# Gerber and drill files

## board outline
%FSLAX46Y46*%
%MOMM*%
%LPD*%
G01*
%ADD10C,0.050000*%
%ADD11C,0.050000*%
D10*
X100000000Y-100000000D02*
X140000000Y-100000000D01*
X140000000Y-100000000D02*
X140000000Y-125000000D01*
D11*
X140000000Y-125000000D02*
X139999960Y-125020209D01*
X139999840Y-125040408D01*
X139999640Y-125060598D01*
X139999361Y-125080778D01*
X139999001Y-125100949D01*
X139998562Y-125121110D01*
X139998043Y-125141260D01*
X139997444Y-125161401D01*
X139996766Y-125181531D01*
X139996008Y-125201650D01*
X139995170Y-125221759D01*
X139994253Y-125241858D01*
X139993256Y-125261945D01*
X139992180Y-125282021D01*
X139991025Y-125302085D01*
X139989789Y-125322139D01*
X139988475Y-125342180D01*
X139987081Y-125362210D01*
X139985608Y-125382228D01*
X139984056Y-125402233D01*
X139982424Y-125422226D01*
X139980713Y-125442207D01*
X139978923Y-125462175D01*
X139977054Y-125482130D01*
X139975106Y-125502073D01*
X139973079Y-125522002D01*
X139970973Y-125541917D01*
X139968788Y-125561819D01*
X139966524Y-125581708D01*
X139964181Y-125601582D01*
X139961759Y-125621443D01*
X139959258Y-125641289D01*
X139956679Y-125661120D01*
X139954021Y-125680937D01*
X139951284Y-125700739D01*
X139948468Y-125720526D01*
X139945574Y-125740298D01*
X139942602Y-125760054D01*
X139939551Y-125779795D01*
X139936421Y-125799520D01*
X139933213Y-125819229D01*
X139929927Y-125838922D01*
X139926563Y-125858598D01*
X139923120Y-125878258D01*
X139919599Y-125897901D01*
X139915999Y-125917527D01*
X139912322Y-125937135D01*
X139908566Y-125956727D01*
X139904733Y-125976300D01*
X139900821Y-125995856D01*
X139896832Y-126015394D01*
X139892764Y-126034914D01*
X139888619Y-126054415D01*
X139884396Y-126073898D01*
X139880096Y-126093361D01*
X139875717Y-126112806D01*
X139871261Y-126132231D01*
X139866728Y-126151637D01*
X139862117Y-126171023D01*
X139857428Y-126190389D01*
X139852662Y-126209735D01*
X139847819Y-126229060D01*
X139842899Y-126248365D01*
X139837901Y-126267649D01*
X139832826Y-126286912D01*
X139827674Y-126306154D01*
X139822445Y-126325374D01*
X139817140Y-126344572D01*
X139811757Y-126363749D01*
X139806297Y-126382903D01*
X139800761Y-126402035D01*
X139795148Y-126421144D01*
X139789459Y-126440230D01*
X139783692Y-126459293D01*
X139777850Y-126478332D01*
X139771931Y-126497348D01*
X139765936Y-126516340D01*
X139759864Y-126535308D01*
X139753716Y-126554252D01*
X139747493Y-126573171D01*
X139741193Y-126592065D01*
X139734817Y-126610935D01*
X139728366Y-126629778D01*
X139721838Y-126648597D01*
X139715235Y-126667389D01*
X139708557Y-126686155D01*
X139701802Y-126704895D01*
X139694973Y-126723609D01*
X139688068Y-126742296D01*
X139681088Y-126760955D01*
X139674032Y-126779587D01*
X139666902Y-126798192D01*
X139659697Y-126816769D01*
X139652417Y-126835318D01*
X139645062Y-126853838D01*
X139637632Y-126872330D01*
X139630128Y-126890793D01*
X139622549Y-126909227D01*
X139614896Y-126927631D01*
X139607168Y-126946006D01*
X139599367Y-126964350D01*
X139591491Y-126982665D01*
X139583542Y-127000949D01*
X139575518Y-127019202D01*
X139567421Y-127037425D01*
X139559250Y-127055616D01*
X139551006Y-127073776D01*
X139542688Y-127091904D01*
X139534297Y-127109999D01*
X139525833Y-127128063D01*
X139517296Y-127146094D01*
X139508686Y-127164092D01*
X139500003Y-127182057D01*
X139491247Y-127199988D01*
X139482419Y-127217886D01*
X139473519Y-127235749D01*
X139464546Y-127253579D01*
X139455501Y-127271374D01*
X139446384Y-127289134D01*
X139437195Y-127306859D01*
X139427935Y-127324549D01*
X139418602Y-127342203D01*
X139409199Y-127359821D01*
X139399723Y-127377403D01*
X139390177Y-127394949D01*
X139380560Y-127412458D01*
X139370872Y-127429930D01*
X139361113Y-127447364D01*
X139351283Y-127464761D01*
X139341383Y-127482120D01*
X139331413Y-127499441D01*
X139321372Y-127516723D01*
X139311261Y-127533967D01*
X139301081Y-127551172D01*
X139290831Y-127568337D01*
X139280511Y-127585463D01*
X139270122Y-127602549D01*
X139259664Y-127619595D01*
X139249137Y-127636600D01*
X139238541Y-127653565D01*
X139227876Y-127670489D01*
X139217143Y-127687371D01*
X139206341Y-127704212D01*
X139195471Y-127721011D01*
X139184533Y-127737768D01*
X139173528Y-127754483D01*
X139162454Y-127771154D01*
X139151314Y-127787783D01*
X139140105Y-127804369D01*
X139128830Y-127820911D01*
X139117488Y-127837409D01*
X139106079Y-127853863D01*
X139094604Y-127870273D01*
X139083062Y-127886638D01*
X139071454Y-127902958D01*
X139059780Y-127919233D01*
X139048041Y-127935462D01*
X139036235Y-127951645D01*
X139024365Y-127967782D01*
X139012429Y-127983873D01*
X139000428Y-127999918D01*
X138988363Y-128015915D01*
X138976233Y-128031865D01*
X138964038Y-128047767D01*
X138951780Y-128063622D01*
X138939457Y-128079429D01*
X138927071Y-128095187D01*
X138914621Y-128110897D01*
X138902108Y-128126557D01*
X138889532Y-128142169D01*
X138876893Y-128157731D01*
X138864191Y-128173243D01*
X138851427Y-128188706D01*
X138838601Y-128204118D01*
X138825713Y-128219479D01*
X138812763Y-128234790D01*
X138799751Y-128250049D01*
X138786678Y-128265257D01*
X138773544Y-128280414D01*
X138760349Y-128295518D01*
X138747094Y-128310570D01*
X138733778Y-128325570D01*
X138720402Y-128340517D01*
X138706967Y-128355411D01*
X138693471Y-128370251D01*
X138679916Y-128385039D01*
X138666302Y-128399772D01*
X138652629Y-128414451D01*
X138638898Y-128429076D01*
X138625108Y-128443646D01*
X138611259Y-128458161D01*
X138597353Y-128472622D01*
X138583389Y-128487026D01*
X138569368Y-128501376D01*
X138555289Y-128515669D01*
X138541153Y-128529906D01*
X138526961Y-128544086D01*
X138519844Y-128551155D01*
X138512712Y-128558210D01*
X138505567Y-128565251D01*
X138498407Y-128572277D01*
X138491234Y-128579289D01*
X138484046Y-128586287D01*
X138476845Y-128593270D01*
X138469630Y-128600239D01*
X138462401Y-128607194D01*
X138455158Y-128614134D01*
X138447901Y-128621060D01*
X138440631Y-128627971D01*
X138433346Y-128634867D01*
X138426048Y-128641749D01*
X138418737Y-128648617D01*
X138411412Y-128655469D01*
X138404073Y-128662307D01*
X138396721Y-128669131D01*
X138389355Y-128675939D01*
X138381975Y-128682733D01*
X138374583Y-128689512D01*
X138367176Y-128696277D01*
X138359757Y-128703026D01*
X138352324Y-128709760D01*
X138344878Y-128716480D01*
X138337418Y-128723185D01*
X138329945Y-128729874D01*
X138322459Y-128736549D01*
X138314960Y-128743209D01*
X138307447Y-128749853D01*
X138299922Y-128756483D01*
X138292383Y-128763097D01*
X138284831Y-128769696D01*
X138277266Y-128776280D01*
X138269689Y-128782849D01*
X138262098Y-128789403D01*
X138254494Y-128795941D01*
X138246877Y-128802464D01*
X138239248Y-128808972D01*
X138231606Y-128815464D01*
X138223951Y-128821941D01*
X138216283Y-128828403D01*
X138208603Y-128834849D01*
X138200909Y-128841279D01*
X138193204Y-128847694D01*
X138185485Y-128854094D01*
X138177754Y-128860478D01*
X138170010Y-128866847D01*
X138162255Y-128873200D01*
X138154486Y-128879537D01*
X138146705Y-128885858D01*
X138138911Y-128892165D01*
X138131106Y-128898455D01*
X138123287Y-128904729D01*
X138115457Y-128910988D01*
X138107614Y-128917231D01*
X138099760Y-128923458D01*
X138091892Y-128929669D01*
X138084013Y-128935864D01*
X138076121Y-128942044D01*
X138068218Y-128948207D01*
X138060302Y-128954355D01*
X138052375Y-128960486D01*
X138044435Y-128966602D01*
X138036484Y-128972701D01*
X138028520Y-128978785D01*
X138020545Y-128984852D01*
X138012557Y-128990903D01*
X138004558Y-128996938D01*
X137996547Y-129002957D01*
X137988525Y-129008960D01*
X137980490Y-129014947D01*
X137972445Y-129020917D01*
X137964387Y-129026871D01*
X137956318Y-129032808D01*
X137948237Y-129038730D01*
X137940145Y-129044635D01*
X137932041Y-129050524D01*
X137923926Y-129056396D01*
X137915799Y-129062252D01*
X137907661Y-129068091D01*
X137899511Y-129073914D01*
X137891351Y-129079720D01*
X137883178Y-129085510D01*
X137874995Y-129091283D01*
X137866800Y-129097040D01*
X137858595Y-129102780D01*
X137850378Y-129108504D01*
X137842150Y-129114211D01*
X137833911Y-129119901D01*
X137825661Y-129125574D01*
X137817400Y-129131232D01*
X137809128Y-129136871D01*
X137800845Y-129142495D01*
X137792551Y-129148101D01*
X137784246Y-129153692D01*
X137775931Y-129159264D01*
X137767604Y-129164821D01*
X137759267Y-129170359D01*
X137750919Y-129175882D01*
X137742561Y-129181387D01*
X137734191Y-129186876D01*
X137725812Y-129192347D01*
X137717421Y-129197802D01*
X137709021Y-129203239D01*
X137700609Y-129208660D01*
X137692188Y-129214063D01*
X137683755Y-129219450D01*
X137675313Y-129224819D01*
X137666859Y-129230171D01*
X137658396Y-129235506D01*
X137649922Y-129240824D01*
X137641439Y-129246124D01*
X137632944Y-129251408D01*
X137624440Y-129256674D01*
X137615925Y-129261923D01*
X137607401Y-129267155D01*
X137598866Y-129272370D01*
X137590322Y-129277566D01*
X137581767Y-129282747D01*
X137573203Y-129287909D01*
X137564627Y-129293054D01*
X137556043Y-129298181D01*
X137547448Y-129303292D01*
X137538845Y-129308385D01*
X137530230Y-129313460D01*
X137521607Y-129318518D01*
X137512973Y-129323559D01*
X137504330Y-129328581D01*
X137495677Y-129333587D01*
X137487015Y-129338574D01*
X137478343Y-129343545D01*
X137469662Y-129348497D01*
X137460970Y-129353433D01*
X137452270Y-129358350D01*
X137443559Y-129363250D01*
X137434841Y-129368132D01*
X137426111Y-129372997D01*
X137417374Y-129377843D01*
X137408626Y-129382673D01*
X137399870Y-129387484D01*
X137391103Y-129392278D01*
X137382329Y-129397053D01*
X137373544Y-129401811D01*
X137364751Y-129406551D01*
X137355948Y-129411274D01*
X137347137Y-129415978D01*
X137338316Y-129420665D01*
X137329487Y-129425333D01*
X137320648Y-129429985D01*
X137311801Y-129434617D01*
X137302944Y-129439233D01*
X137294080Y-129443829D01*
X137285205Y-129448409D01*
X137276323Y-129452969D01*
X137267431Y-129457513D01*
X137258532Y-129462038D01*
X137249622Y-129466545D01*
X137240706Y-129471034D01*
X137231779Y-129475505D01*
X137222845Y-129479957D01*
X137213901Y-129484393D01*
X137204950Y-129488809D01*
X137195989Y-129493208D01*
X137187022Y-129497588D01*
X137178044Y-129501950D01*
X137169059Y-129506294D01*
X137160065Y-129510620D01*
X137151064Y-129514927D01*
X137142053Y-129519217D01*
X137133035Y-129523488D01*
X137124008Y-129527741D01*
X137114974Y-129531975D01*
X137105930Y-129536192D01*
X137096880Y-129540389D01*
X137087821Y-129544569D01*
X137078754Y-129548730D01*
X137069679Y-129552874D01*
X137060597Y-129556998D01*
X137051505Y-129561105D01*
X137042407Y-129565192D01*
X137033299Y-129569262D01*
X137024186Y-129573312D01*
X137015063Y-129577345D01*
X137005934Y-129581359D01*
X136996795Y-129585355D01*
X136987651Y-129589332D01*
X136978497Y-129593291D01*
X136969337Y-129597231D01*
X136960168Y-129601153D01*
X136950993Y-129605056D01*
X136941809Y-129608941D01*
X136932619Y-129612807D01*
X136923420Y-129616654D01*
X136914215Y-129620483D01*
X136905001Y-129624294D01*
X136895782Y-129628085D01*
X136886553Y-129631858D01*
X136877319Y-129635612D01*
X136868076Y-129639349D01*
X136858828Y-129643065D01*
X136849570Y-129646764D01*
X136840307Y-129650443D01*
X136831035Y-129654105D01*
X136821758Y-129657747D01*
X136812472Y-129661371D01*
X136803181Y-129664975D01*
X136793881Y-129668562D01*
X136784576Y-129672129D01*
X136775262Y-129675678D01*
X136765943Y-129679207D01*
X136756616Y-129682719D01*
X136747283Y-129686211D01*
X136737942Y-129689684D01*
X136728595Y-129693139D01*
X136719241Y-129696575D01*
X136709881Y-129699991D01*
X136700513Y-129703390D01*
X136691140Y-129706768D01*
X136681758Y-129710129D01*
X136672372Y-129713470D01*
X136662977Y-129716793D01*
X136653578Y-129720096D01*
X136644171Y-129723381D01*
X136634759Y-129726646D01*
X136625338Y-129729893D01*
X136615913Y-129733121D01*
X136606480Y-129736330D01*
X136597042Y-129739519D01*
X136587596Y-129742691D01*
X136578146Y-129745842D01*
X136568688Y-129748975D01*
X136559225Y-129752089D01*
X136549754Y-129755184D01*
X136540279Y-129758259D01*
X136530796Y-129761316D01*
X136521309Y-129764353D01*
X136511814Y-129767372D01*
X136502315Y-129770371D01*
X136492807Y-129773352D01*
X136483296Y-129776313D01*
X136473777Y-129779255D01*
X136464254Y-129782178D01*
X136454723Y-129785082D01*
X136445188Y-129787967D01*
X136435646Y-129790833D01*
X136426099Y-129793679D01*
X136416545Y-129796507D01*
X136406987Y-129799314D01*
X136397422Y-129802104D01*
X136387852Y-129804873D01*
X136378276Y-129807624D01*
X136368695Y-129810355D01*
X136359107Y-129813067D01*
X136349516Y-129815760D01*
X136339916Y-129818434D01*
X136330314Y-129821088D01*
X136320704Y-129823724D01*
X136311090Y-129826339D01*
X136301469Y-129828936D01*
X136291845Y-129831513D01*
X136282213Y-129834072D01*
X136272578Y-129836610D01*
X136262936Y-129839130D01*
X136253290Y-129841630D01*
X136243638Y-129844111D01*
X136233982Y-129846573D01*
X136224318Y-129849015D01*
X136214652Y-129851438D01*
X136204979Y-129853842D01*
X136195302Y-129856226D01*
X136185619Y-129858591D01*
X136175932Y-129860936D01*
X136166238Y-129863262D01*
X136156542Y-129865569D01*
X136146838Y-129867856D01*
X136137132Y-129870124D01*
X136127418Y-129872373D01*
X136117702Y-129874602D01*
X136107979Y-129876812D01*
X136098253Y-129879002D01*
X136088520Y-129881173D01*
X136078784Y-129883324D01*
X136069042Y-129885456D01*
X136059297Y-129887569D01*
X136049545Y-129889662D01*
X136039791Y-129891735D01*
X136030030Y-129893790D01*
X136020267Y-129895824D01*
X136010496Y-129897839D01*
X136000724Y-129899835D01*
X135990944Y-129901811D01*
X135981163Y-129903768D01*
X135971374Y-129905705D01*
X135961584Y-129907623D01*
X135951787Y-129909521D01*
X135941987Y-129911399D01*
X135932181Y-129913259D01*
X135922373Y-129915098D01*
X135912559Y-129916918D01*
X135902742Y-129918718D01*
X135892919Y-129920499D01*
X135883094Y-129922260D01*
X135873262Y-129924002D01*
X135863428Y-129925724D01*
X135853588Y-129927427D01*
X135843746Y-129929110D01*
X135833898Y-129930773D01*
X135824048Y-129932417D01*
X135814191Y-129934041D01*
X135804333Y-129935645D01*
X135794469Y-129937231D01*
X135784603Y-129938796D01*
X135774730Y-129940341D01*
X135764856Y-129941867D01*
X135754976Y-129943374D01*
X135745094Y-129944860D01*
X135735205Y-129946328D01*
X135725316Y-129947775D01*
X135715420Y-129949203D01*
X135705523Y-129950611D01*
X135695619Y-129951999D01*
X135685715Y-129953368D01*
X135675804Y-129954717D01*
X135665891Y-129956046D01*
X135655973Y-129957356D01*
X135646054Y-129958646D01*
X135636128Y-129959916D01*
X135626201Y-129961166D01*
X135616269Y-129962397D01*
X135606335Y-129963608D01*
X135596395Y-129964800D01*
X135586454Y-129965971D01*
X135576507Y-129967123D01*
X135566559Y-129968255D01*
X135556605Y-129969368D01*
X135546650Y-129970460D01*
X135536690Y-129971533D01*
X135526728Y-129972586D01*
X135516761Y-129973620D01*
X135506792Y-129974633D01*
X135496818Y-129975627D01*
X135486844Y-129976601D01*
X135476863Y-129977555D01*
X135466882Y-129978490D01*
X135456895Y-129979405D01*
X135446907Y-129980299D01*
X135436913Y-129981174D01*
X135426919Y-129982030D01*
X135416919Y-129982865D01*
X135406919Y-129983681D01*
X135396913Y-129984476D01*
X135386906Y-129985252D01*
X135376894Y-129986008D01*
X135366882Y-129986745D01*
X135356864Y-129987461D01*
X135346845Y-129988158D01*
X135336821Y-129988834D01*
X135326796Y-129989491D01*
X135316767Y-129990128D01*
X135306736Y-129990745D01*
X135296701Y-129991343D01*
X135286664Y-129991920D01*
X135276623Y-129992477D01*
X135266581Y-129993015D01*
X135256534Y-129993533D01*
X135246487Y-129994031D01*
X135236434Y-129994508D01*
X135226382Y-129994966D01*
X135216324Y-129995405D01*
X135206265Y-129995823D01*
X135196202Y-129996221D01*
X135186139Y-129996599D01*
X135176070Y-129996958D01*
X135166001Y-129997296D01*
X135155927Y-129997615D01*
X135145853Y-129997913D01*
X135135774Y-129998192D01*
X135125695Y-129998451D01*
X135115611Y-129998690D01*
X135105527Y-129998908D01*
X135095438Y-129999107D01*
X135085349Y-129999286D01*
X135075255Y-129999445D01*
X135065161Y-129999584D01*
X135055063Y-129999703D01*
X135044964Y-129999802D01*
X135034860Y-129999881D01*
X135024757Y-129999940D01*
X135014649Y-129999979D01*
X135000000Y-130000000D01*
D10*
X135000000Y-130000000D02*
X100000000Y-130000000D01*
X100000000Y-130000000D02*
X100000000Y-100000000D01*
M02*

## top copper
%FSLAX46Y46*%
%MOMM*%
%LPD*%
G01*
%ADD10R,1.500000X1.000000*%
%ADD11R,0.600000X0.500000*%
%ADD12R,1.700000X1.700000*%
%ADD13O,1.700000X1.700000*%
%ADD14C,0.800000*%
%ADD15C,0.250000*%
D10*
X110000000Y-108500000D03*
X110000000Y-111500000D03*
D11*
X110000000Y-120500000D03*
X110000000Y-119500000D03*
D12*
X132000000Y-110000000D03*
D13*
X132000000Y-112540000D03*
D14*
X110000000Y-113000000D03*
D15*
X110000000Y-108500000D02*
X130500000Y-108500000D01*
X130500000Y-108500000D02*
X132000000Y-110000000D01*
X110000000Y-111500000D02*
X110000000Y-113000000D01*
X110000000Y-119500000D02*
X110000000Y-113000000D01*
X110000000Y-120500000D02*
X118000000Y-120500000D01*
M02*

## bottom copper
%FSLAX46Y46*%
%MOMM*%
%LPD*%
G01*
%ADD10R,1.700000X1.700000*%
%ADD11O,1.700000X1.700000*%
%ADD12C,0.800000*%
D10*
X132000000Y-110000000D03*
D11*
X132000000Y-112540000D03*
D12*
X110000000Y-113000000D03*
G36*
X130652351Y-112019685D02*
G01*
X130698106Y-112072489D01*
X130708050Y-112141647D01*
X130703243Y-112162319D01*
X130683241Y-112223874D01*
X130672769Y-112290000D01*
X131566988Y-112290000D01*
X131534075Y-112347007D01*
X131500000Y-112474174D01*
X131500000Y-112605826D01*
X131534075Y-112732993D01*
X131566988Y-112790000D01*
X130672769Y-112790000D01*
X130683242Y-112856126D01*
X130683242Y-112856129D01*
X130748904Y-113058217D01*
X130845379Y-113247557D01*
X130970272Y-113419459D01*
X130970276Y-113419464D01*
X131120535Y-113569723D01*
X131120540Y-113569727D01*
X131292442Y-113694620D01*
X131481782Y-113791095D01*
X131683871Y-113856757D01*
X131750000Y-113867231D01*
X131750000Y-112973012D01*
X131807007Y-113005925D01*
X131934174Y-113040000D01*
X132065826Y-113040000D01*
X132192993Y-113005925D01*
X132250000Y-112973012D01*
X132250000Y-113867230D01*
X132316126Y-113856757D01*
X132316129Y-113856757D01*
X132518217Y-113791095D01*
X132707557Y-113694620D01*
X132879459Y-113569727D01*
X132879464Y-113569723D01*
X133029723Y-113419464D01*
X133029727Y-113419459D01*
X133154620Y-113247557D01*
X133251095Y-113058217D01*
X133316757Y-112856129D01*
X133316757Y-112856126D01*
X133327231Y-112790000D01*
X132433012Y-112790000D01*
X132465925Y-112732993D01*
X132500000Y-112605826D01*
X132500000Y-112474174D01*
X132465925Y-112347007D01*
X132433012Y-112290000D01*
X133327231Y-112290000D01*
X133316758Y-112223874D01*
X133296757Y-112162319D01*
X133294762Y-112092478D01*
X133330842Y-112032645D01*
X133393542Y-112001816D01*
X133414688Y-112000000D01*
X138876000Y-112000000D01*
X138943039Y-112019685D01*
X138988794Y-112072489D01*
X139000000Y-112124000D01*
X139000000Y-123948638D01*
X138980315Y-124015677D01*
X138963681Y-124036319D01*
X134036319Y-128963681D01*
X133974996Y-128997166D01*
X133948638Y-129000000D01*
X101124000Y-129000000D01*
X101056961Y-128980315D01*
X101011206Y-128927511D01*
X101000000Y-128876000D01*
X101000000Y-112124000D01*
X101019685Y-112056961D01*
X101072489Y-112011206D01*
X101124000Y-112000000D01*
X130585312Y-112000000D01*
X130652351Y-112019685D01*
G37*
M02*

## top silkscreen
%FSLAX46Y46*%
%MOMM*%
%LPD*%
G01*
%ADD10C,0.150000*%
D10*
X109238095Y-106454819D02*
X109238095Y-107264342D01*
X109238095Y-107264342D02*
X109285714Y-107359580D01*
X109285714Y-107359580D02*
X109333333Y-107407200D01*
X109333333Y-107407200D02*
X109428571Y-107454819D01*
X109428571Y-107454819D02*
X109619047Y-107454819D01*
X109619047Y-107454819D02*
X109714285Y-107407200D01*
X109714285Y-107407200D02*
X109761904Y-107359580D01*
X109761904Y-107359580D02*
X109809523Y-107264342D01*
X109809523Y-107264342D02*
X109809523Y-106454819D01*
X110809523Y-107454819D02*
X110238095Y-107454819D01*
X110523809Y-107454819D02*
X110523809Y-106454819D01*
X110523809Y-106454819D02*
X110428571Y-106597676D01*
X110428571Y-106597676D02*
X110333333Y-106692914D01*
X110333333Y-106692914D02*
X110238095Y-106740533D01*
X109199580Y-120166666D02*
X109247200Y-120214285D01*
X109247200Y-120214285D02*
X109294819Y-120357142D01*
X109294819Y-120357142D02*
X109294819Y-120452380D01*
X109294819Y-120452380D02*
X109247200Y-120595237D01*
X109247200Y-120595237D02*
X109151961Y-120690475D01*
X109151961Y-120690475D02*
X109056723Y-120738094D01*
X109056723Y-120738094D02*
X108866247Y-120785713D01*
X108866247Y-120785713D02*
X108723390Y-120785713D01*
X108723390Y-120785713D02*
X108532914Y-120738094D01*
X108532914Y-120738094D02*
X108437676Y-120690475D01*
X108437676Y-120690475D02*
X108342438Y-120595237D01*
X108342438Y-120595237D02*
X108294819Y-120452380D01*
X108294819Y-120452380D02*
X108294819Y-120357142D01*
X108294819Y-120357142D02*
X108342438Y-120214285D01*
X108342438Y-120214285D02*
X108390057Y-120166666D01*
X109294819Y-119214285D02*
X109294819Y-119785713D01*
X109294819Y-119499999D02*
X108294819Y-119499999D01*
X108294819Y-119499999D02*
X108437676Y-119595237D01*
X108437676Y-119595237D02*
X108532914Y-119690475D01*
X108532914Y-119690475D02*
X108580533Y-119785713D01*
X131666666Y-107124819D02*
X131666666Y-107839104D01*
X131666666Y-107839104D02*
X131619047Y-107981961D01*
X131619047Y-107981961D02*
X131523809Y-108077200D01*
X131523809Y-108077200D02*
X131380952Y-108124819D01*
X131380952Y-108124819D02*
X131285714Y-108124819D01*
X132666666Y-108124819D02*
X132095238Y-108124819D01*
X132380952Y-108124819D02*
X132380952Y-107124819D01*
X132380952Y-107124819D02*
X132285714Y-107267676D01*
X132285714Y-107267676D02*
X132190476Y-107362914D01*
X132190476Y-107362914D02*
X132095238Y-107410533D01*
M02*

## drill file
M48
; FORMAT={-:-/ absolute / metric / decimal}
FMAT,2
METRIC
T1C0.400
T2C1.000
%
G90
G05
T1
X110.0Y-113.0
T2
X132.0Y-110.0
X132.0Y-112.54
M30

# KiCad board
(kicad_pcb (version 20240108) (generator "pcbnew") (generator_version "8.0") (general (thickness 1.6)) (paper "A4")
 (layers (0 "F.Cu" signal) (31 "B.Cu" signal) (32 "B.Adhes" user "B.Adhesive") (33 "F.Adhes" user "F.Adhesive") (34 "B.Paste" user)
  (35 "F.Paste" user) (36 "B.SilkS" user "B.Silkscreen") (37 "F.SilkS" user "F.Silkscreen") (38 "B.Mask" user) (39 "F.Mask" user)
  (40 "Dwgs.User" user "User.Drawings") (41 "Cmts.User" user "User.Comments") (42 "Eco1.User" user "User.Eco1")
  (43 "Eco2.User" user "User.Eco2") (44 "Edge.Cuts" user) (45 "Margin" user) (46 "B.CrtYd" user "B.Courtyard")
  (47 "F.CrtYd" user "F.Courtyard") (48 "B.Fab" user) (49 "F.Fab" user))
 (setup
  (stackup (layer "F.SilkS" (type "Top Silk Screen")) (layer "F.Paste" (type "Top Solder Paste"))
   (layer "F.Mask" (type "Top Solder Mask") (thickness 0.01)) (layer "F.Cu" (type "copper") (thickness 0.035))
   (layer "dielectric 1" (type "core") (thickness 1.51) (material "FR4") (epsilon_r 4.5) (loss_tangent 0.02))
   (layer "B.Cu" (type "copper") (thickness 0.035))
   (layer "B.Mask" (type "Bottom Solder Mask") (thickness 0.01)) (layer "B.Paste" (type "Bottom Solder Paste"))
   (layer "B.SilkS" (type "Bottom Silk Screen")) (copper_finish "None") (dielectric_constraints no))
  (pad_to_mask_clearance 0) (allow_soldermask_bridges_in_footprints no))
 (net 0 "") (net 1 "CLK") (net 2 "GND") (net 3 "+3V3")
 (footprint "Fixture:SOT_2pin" (layer "F.Cu") (at 110 110)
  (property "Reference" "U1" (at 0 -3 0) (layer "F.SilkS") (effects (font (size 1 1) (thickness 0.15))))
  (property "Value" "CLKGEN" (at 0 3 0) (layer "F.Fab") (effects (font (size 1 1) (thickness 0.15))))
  (pad "1" smd rect (at 0 -1.5) (size 1.5 1) (layers "F.Cu" "F.Paste" "F.Mask") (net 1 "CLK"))
  (pad "2" smd rect (at 0 1.5) (size 1.5 1) (layers "F.Cu" "F.Paste" "F.Mask") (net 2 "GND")))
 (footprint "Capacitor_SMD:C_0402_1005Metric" (layer "F.Cu") (at 110 120 90)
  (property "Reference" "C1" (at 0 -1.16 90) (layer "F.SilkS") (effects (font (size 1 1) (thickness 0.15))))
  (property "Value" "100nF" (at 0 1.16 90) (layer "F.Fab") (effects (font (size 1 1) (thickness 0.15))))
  (pad "1" smd rect (at -0.5 0 90) (size 0.5 0.6) (layers "F.Cu" "F.Paste" "F.Mask") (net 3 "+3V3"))
  (pad "2" smd rect (at 0.5 0 90) (size 0.5 0.6) (layers "F.Cu" "F.Paste" "F.Mask") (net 2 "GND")))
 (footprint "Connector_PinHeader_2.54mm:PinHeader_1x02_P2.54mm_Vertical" (layer "F.Cu") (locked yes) (at 132 110)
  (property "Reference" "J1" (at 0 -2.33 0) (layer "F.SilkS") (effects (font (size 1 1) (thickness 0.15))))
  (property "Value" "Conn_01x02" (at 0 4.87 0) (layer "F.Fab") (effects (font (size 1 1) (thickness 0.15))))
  (pad "1" thru_hole rect (at 0 0) (size 1.7 1.7) (drill 1) (layers "*.Cu" "*.Mask") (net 1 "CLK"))
  (pad "2" thru_hole oval (at 0 2.54) (size 1.7 1.7) (drill 1) (layers "*.Cu" "*.Mask") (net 2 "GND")))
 (gr_line (start 100 100) (end 140 100) (stroke (width 0.05) (type default)) (layer "Edge.Cuts"))
 (gr_line (start 140 100) (end 140 125) (stroke (width 0.05) (type default)) (layer "Edge.Cuts"))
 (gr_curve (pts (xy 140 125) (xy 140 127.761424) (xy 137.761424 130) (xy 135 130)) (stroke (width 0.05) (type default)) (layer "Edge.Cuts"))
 (gr_line (start 135 130) (end 100 130) (stroke (width 0.05) (type default)) (layer "Edge.Cuts"))
 (gr_line (start 100 130) (end 100 100) (stroke (width 0.05) (type default)) (layer "Edge.Cuts"))
 (segment (start 110 108.5) (end 130.5 108.5) (width 0.25) (layer "F.Cu") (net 1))
 (segment (start 130.5 108.5) (end 132 110) (width 0.25) (layer "F.Cu") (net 1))
 (segment (start 110 111.5) (end 110 113) (width 0.25) (layer "F.Cu") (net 2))
 (segment (start 110 119.5) (end 110 113) (width 0.25) (layer "F.Cu") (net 2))
 (segment (start 110 120.5) (end 118 120.5) (width 0.25) (layer "F.Cu") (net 3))
 (via (at 110 113) (size 0.8) (drill 0.4) (layers "F.Cu" "B.Cu") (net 2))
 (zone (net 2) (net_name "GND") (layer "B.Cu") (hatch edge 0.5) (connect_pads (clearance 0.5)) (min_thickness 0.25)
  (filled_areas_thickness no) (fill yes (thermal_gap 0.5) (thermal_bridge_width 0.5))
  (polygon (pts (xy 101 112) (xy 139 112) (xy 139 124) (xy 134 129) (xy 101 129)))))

